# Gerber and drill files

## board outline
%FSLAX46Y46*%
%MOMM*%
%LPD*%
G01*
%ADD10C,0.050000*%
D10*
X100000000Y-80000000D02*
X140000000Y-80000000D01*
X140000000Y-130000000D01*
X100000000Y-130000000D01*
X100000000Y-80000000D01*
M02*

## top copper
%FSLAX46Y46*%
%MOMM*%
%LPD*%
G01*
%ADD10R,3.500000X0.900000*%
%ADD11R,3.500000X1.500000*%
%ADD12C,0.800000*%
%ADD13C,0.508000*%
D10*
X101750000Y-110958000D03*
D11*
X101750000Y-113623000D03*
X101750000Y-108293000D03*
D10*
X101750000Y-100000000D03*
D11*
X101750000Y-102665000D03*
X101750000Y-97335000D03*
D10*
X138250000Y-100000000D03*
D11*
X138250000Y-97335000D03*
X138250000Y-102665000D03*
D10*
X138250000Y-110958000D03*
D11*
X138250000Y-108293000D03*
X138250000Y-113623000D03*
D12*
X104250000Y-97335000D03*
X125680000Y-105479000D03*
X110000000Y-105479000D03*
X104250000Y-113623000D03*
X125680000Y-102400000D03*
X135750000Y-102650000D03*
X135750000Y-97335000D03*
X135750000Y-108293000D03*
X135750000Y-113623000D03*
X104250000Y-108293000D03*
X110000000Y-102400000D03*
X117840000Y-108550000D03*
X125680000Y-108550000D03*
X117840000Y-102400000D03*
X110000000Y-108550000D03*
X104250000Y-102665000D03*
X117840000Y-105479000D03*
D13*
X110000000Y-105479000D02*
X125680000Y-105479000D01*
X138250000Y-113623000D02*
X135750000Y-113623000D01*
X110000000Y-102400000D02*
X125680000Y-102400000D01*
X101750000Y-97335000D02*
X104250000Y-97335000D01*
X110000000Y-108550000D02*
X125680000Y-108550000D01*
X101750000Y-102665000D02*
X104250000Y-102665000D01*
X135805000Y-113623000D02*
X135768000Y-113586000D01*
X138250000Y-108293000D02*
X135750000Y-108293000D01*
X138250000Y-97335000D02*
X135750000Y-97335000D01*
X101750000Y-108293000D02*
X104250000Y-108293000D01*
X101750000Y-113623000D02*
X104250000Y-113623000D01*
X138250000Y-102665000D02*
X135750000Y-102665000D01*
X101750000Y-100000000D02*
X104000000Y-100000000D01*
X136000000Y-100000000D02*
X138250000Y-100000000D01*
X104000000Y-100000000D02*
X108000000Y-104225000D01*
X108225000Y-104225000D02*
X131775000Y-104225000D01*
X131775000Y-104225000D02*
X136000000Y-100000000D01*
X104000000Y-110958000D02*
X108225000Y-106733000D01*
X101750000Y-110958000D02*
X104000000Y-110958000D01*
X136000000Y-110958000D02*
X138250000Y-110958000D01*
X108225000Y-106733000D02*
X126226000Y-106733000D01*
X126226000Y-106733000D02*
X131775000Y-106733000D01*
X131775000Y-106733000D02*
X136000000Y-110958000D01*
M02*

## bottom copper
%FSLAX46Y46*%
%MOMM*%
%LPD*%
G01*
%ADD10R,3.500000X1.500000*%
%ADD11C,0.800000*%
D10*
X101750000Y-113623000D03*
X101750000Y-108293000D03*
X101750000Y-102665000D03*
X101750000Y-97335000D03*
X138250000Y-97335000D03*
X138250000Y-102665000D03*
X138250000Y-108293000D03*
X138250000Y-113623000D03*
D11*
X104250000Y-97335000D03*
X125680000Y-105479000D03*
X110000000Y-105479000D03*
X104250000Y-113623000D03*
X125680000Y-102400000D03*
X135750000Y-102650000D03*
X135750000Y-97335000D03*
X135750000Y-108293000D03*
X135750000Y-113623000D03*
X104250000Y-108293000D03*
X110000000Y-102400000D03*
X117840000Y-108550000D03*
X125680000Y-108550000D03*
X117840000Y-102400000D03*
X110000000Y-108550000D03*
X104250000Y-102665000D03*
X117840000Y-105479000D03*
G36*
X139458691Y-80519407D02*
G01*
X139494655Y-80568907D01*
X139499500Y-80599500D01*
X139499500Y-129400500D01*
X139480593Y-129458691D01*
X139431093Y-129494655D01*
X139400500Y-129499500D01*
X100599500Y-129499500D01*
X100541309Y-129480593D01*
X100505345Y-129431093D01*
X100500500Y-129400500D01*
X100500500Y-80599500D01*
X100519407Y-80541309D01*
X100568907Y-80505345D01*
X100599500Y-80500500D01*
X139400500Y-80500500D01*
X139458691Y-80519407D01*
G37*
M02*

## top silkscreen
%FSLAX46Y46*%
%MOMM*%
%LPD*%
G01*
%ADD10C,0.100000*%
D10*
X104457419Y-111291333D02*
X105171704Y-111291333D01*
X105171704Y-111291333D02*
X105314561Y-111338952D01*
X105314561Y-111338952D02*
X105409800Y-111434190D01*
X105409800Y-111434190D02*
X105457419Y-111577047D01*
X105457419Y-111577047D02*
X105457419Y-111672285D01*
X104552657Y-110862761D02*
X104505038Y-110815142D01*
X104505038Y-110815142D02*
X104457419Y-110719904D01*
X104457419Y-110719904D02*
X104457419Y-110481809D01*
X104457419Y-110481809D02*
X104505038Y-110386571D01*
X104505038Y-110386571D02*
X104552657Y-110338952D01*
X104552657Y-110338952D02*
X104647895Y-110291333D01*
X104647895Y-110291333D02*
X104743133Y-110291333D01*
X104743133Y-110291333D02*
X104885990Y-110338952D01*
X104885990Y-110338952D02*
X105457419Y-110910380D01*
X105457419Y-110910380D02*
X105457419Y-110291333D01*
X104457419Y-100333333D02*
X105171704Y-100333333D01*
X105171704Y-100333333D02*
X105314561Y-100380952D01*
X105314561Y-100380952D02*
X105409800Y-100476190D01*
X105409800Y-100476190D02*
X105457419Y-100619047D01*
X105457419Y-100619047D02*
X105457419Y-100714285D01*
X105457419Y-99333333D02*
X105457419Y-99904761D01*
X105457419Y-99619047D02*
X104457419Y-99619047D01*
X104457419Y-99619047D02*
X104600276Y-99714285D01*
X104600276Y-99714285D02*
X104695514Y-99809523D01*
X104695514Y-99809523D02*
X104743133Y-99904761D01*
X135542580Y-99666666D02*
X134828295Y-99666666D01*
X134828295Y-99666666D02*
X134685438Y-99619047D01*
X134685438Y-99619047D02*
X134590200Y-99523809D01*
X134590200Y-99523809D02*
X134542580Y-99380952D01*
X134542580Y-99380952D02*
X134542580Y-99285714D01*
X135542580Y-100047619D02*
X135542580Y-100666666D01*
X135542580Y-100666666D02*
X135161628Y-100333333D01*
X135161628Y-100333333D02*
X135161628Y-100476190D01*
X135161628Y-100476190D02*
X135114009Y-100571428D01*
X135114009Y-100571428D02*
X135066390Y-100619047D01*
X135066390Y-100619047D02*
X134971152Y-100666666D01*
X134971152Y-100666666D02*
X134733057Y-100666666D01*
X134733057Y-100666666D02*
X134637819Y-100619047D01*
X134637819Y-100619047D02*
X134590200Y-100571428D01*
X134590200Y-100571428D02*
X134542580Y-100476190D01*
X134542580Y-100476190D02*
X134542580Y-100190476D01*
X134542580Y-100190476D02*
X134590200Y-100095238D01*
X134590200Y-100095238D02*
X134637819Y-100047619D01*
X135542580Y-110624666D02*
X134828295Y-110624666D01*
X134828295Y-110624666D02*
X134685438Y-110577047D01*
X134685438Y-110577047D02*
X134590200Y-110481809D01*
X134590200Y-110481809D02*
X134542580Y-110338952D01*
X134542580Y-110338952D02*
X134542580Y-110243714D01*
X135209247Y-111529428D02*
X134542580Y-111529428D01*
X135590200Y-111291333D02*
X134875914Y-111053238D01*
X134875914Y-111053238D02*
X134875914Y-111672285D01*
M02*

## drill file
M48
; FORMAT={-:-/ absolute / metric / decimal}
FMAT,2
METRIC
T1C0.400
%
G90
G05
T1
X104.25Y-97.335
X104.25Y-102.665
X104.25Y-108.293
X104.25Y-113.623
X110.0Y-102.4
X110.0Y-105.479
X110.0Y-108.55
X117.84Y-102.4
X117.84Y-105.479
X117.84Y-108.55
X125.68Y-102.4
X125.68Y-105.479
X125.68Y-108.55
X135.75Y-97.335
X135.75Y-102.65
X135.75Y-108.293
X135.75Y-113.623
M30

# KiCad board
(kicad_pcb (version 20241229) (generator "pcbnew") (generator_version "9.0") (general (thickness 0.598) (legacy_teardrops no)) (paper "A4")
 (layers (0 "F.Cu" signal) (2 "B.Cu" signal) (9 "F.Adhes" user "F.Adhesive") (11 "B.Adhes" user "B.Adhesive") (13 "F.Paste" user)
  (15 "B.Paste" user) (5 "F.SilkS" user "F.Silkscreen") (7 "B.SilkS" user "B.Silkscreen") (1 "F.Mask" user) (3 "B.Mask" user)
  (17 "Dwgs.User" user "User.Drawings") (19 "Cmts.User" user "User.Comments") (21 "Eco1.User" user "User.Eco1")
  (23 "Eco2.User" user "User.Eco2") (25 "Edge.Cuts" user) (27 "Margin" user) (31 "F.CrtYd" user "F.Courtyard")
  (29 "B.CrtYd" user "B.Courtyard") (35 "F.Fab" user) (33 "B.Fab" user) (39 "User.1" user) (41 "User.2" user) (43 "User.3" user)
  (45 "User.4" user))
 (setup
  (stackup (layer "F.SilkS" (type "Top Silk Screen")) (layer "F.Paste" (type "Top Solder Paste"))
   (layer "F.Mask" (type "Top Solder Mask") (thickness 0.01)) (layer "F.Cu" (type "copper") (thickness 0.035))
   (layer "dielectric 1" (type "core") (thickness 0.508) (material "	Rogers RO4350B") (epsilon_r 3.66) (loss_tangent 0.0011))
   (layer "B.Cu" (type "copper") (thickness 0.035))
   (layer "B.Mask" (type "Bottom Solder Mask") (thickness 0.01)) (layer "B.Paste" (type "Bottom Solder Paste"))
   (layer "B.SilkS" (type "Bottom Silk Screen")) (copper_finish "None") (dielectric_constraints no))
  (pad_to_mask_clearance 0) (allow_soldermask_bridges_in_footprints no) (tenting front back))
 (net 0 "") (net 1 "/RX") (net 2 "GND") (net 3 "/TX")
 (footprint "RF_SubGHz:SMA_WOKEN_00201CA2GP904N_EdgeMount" (layer "F.Cu") (at 100 110.958 90)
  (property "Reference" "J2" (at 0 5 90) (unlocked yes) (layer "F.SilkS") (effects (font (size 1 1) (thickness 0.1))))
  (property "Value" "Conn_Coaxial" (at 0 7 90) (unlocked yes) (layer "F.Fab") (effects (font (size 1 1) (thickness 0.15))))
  (pad "1" smd rect (at 0 1.75 90) (size 0.9 3.5) (layers "F.Cu" "F.Mask") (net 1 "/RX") (thermal_bridge_angle 45))
  (pad "2" smd rect (at -2.665 1.75 90) (size 1.5 3.5) (layers "F.Cu" "F.Mask") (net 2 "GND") (thermal_bridge_angle 45))
  (pad "2" smd rect (at -2.665 1.75 90) (size 1.5 3.5) (layers "B.Cu" "B.Mask") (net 2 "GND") (thermal_bridge_angle 45))
  (pad "2" smd rect (at 2.665 1.75 90) (size 1.5 3.5) (layers "F.Cu" "F.Mask") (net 2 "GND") (thermal_bridge_angle 45))
  (pad "2" smd rect (at 2.665 1.75 90) (size 1.5 3.5) (layers "B.Cu" "B.Mask") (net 2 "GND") (thermal_bridge_angle 45)))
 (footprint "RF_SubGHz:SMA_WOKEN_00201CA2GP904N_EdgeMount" (layer "F.Cu") (at 100 100 90)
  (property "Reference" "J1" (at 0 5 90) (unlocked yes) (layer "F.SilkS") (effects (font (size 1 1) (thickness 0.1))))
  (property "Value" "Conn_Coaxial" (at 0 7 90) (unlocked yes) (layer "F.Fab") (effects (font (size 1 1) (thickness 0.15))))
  (pad "1" smd rect (at 0 1.75 90) (size 0.9 3.5) (layers "F.Cu" "F.Mask") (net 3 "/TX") (thermal_bridge_angle 45))
  (pad "2" smd rect (at -2.665 1.75 90) (size 1.5 3.5) (layers "F.Cu" "F.Mask") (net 2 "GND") (thermal_bridge_angle 45))
  (pad "2" smd rect (at -2.665 1.75 90) (size 1.5 3.5) (layers "B.Cu" "B.Mask") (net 2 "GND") (thermal_bridge_angle 45))
  (pad "2" smd rect (at 2.665 1.75 90) (size 1.5 3.5) (layers "F.Cu" "F.Mask") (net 2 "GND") (thermal_bridge_angle 45))
  (pad "2" smd rect (at 2.665 1.75 90) (size 1.5 3.5) (layers "B.Cu" "B.Mask") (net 2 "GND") (thermal_bridge_angle 45)))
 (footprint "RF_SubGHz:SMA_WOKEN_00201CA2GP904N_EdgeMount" (layer "F.Cu") (at 140 100 -90)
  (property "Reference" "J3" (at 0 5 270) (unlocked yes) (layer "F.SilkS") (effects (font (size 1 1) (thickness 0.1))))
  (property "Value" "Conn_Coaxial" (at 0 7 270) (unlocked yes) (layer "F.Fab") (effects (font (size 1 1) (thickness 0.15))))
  (pad "1" smd rect (at 0 1.75 270) (size 0.9 3.5) (layers "F.Cu" "F.Mask") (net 3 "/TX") (thermal_bridge_angle 45))
  (pad "2" smd rect (at -2.665 1.75 270) (size 1.5 3.5) (layers "F.Cu" "F.Mask") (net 2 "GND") (thermal_bridge_angle 45))
  (pad "2" smd rect (at -2.665 1.75 270) (size 1.5 3.5) (layers "B.Cu" "B.Mask") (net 2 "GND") (thermal_bridge_angle 45))
  (pad "2" smd rect (at 2.665 1.75 270) (size 1.5 3.5) (layers "F.Cu" "F.Mask") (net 2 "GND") (thermal_bridge_angle 45))
  (pad "2" smd rect (at 2.665 1.75 270) (size 1.5 3.5) (layers "B.Cu" "B.Mask") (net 2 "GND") (thermal_bridge_angle 45)))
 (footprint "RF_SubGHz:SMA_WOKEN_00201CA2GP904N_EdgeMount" (layer "F.Cu") (at 140 110.958 -90)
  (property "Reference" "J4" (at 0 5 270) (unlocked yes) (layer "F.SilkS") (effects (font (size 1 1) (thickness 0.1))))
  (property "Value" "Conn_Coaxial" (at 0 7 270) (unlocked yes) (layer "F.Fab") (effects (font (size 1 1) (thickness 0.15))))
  (pad "1" smd rect (at 0 1.75 270) (size 0.9 3.5) (layers "F.Cu" "F.Mask") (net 1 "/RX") (thermal_bridge_angle 45))
  (pad "2" smd rect (at -2.665 1.75 270) (size 1.5 3.5) (layers "F.Cu" "F.Mask") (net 2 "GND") (thermal_bridge_angle 45))
  (pad "2" smd rect (at -2.665 1.75 270) (size 1.5 3.5) (layers "B.Cu" "B.Mask") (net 2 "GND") (thermal_bridge_angle 45))
  (pad "2" smd rect (at 2.665 1.75 270) (size 1.5 3.5) (layers "F.Cu" "F.Mask") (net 2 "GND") (thermal_bridge_angle 45))
  (pad "2" smd rect (at 2.665 1.75 270) (size 1.5 3.5) (layers "B.Cu" "B.Mask") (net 2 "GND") (thermal_bridge_angle 45)))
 (gr_rect (start 100 80) (end 140 130) (stroke (width 0.05) (type solid)) (fill no) (layer "Edge.Cuts"))
 (segment (start 110 105.479) (end 125.68 105.479) (width 0.508) (layer "F.Cu") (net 2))
 (segment (start 138.25 113.623) (end 135.75 113.623) (width 0.508) (layer "F.Cu") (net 2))
 (segment (start 110 102.4) (end 125.68 102.4) (width 0.508) (layer "F.Cu") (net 2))
 (segment (start 101.75 97.335) (end 104.25 97.335) (width 0.508) (layer "F.Cu") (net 2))
 (segment (start 110 108.55) (end 125.68 108.55) (width 0.508) (layer "F.Cu") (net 2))
 (segment (start 101.75 102.665) (end 104.25 102.665) (width 0.508) (layer "F.Cu") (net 2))
 (segment (start 135.805 113.623) (end 135.768 113.586) (width 0.508) (layer "F.Cu") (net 2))
 (segment (start 138.25 108.293) (end 135.75 108.293) (width 0.508) (layer "F.Cu") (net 2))
 (segment (start 138.25 97.335) (end 135.75 97.335) (width 0.508) (layer "F.Cu") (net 2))
 (segment (start 101.75 108.293) (end 104.25 108.293) (width 0.508) (layer "F.Cu") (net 2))
 (segment (start 101.75 113.623) (end 104.25 113.623) (width 0.508) (layer "F.Cu") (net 2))
 (segment (start 138.25 102.665) (end 135.75 102.665) (width 0.508) (layer "F.Cu") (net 2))
 (via (at 104.25 97.335) (size 0.8) (drill 0.4) (layers "F.Cu" "B.Cu") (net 2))
 (via (at 125.68 105.479) (size 0.8) (drill 0.4) (layers "F.Cu" "B.Cu") (free yes) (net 2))
 (via (at 110 105.479) (size 0.8) (drill 0.4) (layers "F.Cu" "B.Cu") (free yes) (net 2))
 (via (at 104.25 113.623) (size 0.8) (drill 0.4) (layers "F.Cu" "B.Cu") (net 2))
 (via (at 125.68 102.4) (size 0.8) (drill 0.4) (layers "F.Cu" "B.Cu") (free yes) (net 2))
 (via (at 135.75 102.65) (size 0.8) (drill 0.4) (layers "F.Cu" "B.Cu") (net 2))
 (via (at 135.75 97.335) (size 0.8) (drill 0.4) (layers "F.Cu" "B.Cu") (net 2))
 (via (at 135.75 108.293) (size 0.8) (drill 0.4) (layers "F.Cu" "B.Cu") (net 2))
 (via (at 135.75 113.623) (size 0.8) (drill 0.4) (layers "F.Cu" "B.Cu") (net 2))
 (via (at 104.25 108.293) (size 0.8) (drill 0.4) (layers "F.Cu" "B.Cu") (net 2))
 (via (at 110 102.4) (size 0.8) (drill 0.4) (layers "F.Cu" "B.Cu") (free yes) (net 2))
 (via (at 117.84 108.55) (size 0.8) (drill 0.4) (layers "F.Cu" "B.Cu") (free yes) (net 2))
 (via (at 125.68 108.55) (size 0.8) (drill 0.4) (layers "F.Cu" "B.Cu") (free yes) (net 2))
 (via (at 117.84 102.4) (size 0.8) (drill 0.4) (layers "F.Cu" "B.Cu") (free yes) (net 2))
 (via (at 110 108.55) (size 0.8) (drill 0.4) (layers "F.Cu" "B.Cu") (free yes) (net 2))
 (via (at 104.25 102.665) (size 0.8) (drill 0.4) (layers "F.Cu" "B.Cu") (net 2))
 (via (at 117.84 105.479) (size 0.8) (drill 0.4) (layers "F.Cu" "B.Cu") (free yes) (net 2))
 (segment (start 101.75 100) (end 104 100) (width 0.508) (layer "F.Cu") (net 3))
 (segment (start 136 100) (end 138.25 100) (width 0.508) (layer "F.Cu") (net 3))
 (segment (start 104 100) (end 108 104.225) (width 0.508) (layer "F.Cu") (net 3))
 (segment (start 108.225 104.225) (end 131.775 104.225) (width 0.508) (layer "F.Cu") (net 3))
 (segment (start 131.775 104.225) (end 136 100) (width 0.508) (layer "F.Cu") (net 3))
 (segment (start 104 110.958) (end 108.225 106.733) (width 0.508) (layer "F.Cu") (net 1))
 (segment (start 101.75 110.958) (end 104 110.958) (width 0.508) (layer "F.Cu") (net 1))
 (segment (start 136 110.958) (end 138.25 110.958) (width 0.508) (layer "F.Cu") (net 1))
 (segment (start 108.225 106.733) (end 126.226 106.733) (width 0.508) (layer "F.Cu") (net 1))
 (segment (start 126.226 106.733) (end 131.775 106.733) (width 0.508) (layer "F.Cu") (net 1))
 (segment (start 131.775 106.733) (end 136 110.958) (width 0.508) (layer "F.Cu") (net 1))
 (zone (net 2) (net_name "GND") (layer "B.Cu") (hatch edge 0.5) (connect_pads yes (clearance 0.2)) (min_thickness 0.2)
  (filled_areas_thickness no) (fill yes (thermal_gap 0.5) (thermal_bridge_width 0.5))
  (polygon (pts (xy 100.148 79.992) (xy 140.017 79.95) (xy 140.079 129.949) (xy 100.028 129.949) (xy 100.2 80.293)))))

